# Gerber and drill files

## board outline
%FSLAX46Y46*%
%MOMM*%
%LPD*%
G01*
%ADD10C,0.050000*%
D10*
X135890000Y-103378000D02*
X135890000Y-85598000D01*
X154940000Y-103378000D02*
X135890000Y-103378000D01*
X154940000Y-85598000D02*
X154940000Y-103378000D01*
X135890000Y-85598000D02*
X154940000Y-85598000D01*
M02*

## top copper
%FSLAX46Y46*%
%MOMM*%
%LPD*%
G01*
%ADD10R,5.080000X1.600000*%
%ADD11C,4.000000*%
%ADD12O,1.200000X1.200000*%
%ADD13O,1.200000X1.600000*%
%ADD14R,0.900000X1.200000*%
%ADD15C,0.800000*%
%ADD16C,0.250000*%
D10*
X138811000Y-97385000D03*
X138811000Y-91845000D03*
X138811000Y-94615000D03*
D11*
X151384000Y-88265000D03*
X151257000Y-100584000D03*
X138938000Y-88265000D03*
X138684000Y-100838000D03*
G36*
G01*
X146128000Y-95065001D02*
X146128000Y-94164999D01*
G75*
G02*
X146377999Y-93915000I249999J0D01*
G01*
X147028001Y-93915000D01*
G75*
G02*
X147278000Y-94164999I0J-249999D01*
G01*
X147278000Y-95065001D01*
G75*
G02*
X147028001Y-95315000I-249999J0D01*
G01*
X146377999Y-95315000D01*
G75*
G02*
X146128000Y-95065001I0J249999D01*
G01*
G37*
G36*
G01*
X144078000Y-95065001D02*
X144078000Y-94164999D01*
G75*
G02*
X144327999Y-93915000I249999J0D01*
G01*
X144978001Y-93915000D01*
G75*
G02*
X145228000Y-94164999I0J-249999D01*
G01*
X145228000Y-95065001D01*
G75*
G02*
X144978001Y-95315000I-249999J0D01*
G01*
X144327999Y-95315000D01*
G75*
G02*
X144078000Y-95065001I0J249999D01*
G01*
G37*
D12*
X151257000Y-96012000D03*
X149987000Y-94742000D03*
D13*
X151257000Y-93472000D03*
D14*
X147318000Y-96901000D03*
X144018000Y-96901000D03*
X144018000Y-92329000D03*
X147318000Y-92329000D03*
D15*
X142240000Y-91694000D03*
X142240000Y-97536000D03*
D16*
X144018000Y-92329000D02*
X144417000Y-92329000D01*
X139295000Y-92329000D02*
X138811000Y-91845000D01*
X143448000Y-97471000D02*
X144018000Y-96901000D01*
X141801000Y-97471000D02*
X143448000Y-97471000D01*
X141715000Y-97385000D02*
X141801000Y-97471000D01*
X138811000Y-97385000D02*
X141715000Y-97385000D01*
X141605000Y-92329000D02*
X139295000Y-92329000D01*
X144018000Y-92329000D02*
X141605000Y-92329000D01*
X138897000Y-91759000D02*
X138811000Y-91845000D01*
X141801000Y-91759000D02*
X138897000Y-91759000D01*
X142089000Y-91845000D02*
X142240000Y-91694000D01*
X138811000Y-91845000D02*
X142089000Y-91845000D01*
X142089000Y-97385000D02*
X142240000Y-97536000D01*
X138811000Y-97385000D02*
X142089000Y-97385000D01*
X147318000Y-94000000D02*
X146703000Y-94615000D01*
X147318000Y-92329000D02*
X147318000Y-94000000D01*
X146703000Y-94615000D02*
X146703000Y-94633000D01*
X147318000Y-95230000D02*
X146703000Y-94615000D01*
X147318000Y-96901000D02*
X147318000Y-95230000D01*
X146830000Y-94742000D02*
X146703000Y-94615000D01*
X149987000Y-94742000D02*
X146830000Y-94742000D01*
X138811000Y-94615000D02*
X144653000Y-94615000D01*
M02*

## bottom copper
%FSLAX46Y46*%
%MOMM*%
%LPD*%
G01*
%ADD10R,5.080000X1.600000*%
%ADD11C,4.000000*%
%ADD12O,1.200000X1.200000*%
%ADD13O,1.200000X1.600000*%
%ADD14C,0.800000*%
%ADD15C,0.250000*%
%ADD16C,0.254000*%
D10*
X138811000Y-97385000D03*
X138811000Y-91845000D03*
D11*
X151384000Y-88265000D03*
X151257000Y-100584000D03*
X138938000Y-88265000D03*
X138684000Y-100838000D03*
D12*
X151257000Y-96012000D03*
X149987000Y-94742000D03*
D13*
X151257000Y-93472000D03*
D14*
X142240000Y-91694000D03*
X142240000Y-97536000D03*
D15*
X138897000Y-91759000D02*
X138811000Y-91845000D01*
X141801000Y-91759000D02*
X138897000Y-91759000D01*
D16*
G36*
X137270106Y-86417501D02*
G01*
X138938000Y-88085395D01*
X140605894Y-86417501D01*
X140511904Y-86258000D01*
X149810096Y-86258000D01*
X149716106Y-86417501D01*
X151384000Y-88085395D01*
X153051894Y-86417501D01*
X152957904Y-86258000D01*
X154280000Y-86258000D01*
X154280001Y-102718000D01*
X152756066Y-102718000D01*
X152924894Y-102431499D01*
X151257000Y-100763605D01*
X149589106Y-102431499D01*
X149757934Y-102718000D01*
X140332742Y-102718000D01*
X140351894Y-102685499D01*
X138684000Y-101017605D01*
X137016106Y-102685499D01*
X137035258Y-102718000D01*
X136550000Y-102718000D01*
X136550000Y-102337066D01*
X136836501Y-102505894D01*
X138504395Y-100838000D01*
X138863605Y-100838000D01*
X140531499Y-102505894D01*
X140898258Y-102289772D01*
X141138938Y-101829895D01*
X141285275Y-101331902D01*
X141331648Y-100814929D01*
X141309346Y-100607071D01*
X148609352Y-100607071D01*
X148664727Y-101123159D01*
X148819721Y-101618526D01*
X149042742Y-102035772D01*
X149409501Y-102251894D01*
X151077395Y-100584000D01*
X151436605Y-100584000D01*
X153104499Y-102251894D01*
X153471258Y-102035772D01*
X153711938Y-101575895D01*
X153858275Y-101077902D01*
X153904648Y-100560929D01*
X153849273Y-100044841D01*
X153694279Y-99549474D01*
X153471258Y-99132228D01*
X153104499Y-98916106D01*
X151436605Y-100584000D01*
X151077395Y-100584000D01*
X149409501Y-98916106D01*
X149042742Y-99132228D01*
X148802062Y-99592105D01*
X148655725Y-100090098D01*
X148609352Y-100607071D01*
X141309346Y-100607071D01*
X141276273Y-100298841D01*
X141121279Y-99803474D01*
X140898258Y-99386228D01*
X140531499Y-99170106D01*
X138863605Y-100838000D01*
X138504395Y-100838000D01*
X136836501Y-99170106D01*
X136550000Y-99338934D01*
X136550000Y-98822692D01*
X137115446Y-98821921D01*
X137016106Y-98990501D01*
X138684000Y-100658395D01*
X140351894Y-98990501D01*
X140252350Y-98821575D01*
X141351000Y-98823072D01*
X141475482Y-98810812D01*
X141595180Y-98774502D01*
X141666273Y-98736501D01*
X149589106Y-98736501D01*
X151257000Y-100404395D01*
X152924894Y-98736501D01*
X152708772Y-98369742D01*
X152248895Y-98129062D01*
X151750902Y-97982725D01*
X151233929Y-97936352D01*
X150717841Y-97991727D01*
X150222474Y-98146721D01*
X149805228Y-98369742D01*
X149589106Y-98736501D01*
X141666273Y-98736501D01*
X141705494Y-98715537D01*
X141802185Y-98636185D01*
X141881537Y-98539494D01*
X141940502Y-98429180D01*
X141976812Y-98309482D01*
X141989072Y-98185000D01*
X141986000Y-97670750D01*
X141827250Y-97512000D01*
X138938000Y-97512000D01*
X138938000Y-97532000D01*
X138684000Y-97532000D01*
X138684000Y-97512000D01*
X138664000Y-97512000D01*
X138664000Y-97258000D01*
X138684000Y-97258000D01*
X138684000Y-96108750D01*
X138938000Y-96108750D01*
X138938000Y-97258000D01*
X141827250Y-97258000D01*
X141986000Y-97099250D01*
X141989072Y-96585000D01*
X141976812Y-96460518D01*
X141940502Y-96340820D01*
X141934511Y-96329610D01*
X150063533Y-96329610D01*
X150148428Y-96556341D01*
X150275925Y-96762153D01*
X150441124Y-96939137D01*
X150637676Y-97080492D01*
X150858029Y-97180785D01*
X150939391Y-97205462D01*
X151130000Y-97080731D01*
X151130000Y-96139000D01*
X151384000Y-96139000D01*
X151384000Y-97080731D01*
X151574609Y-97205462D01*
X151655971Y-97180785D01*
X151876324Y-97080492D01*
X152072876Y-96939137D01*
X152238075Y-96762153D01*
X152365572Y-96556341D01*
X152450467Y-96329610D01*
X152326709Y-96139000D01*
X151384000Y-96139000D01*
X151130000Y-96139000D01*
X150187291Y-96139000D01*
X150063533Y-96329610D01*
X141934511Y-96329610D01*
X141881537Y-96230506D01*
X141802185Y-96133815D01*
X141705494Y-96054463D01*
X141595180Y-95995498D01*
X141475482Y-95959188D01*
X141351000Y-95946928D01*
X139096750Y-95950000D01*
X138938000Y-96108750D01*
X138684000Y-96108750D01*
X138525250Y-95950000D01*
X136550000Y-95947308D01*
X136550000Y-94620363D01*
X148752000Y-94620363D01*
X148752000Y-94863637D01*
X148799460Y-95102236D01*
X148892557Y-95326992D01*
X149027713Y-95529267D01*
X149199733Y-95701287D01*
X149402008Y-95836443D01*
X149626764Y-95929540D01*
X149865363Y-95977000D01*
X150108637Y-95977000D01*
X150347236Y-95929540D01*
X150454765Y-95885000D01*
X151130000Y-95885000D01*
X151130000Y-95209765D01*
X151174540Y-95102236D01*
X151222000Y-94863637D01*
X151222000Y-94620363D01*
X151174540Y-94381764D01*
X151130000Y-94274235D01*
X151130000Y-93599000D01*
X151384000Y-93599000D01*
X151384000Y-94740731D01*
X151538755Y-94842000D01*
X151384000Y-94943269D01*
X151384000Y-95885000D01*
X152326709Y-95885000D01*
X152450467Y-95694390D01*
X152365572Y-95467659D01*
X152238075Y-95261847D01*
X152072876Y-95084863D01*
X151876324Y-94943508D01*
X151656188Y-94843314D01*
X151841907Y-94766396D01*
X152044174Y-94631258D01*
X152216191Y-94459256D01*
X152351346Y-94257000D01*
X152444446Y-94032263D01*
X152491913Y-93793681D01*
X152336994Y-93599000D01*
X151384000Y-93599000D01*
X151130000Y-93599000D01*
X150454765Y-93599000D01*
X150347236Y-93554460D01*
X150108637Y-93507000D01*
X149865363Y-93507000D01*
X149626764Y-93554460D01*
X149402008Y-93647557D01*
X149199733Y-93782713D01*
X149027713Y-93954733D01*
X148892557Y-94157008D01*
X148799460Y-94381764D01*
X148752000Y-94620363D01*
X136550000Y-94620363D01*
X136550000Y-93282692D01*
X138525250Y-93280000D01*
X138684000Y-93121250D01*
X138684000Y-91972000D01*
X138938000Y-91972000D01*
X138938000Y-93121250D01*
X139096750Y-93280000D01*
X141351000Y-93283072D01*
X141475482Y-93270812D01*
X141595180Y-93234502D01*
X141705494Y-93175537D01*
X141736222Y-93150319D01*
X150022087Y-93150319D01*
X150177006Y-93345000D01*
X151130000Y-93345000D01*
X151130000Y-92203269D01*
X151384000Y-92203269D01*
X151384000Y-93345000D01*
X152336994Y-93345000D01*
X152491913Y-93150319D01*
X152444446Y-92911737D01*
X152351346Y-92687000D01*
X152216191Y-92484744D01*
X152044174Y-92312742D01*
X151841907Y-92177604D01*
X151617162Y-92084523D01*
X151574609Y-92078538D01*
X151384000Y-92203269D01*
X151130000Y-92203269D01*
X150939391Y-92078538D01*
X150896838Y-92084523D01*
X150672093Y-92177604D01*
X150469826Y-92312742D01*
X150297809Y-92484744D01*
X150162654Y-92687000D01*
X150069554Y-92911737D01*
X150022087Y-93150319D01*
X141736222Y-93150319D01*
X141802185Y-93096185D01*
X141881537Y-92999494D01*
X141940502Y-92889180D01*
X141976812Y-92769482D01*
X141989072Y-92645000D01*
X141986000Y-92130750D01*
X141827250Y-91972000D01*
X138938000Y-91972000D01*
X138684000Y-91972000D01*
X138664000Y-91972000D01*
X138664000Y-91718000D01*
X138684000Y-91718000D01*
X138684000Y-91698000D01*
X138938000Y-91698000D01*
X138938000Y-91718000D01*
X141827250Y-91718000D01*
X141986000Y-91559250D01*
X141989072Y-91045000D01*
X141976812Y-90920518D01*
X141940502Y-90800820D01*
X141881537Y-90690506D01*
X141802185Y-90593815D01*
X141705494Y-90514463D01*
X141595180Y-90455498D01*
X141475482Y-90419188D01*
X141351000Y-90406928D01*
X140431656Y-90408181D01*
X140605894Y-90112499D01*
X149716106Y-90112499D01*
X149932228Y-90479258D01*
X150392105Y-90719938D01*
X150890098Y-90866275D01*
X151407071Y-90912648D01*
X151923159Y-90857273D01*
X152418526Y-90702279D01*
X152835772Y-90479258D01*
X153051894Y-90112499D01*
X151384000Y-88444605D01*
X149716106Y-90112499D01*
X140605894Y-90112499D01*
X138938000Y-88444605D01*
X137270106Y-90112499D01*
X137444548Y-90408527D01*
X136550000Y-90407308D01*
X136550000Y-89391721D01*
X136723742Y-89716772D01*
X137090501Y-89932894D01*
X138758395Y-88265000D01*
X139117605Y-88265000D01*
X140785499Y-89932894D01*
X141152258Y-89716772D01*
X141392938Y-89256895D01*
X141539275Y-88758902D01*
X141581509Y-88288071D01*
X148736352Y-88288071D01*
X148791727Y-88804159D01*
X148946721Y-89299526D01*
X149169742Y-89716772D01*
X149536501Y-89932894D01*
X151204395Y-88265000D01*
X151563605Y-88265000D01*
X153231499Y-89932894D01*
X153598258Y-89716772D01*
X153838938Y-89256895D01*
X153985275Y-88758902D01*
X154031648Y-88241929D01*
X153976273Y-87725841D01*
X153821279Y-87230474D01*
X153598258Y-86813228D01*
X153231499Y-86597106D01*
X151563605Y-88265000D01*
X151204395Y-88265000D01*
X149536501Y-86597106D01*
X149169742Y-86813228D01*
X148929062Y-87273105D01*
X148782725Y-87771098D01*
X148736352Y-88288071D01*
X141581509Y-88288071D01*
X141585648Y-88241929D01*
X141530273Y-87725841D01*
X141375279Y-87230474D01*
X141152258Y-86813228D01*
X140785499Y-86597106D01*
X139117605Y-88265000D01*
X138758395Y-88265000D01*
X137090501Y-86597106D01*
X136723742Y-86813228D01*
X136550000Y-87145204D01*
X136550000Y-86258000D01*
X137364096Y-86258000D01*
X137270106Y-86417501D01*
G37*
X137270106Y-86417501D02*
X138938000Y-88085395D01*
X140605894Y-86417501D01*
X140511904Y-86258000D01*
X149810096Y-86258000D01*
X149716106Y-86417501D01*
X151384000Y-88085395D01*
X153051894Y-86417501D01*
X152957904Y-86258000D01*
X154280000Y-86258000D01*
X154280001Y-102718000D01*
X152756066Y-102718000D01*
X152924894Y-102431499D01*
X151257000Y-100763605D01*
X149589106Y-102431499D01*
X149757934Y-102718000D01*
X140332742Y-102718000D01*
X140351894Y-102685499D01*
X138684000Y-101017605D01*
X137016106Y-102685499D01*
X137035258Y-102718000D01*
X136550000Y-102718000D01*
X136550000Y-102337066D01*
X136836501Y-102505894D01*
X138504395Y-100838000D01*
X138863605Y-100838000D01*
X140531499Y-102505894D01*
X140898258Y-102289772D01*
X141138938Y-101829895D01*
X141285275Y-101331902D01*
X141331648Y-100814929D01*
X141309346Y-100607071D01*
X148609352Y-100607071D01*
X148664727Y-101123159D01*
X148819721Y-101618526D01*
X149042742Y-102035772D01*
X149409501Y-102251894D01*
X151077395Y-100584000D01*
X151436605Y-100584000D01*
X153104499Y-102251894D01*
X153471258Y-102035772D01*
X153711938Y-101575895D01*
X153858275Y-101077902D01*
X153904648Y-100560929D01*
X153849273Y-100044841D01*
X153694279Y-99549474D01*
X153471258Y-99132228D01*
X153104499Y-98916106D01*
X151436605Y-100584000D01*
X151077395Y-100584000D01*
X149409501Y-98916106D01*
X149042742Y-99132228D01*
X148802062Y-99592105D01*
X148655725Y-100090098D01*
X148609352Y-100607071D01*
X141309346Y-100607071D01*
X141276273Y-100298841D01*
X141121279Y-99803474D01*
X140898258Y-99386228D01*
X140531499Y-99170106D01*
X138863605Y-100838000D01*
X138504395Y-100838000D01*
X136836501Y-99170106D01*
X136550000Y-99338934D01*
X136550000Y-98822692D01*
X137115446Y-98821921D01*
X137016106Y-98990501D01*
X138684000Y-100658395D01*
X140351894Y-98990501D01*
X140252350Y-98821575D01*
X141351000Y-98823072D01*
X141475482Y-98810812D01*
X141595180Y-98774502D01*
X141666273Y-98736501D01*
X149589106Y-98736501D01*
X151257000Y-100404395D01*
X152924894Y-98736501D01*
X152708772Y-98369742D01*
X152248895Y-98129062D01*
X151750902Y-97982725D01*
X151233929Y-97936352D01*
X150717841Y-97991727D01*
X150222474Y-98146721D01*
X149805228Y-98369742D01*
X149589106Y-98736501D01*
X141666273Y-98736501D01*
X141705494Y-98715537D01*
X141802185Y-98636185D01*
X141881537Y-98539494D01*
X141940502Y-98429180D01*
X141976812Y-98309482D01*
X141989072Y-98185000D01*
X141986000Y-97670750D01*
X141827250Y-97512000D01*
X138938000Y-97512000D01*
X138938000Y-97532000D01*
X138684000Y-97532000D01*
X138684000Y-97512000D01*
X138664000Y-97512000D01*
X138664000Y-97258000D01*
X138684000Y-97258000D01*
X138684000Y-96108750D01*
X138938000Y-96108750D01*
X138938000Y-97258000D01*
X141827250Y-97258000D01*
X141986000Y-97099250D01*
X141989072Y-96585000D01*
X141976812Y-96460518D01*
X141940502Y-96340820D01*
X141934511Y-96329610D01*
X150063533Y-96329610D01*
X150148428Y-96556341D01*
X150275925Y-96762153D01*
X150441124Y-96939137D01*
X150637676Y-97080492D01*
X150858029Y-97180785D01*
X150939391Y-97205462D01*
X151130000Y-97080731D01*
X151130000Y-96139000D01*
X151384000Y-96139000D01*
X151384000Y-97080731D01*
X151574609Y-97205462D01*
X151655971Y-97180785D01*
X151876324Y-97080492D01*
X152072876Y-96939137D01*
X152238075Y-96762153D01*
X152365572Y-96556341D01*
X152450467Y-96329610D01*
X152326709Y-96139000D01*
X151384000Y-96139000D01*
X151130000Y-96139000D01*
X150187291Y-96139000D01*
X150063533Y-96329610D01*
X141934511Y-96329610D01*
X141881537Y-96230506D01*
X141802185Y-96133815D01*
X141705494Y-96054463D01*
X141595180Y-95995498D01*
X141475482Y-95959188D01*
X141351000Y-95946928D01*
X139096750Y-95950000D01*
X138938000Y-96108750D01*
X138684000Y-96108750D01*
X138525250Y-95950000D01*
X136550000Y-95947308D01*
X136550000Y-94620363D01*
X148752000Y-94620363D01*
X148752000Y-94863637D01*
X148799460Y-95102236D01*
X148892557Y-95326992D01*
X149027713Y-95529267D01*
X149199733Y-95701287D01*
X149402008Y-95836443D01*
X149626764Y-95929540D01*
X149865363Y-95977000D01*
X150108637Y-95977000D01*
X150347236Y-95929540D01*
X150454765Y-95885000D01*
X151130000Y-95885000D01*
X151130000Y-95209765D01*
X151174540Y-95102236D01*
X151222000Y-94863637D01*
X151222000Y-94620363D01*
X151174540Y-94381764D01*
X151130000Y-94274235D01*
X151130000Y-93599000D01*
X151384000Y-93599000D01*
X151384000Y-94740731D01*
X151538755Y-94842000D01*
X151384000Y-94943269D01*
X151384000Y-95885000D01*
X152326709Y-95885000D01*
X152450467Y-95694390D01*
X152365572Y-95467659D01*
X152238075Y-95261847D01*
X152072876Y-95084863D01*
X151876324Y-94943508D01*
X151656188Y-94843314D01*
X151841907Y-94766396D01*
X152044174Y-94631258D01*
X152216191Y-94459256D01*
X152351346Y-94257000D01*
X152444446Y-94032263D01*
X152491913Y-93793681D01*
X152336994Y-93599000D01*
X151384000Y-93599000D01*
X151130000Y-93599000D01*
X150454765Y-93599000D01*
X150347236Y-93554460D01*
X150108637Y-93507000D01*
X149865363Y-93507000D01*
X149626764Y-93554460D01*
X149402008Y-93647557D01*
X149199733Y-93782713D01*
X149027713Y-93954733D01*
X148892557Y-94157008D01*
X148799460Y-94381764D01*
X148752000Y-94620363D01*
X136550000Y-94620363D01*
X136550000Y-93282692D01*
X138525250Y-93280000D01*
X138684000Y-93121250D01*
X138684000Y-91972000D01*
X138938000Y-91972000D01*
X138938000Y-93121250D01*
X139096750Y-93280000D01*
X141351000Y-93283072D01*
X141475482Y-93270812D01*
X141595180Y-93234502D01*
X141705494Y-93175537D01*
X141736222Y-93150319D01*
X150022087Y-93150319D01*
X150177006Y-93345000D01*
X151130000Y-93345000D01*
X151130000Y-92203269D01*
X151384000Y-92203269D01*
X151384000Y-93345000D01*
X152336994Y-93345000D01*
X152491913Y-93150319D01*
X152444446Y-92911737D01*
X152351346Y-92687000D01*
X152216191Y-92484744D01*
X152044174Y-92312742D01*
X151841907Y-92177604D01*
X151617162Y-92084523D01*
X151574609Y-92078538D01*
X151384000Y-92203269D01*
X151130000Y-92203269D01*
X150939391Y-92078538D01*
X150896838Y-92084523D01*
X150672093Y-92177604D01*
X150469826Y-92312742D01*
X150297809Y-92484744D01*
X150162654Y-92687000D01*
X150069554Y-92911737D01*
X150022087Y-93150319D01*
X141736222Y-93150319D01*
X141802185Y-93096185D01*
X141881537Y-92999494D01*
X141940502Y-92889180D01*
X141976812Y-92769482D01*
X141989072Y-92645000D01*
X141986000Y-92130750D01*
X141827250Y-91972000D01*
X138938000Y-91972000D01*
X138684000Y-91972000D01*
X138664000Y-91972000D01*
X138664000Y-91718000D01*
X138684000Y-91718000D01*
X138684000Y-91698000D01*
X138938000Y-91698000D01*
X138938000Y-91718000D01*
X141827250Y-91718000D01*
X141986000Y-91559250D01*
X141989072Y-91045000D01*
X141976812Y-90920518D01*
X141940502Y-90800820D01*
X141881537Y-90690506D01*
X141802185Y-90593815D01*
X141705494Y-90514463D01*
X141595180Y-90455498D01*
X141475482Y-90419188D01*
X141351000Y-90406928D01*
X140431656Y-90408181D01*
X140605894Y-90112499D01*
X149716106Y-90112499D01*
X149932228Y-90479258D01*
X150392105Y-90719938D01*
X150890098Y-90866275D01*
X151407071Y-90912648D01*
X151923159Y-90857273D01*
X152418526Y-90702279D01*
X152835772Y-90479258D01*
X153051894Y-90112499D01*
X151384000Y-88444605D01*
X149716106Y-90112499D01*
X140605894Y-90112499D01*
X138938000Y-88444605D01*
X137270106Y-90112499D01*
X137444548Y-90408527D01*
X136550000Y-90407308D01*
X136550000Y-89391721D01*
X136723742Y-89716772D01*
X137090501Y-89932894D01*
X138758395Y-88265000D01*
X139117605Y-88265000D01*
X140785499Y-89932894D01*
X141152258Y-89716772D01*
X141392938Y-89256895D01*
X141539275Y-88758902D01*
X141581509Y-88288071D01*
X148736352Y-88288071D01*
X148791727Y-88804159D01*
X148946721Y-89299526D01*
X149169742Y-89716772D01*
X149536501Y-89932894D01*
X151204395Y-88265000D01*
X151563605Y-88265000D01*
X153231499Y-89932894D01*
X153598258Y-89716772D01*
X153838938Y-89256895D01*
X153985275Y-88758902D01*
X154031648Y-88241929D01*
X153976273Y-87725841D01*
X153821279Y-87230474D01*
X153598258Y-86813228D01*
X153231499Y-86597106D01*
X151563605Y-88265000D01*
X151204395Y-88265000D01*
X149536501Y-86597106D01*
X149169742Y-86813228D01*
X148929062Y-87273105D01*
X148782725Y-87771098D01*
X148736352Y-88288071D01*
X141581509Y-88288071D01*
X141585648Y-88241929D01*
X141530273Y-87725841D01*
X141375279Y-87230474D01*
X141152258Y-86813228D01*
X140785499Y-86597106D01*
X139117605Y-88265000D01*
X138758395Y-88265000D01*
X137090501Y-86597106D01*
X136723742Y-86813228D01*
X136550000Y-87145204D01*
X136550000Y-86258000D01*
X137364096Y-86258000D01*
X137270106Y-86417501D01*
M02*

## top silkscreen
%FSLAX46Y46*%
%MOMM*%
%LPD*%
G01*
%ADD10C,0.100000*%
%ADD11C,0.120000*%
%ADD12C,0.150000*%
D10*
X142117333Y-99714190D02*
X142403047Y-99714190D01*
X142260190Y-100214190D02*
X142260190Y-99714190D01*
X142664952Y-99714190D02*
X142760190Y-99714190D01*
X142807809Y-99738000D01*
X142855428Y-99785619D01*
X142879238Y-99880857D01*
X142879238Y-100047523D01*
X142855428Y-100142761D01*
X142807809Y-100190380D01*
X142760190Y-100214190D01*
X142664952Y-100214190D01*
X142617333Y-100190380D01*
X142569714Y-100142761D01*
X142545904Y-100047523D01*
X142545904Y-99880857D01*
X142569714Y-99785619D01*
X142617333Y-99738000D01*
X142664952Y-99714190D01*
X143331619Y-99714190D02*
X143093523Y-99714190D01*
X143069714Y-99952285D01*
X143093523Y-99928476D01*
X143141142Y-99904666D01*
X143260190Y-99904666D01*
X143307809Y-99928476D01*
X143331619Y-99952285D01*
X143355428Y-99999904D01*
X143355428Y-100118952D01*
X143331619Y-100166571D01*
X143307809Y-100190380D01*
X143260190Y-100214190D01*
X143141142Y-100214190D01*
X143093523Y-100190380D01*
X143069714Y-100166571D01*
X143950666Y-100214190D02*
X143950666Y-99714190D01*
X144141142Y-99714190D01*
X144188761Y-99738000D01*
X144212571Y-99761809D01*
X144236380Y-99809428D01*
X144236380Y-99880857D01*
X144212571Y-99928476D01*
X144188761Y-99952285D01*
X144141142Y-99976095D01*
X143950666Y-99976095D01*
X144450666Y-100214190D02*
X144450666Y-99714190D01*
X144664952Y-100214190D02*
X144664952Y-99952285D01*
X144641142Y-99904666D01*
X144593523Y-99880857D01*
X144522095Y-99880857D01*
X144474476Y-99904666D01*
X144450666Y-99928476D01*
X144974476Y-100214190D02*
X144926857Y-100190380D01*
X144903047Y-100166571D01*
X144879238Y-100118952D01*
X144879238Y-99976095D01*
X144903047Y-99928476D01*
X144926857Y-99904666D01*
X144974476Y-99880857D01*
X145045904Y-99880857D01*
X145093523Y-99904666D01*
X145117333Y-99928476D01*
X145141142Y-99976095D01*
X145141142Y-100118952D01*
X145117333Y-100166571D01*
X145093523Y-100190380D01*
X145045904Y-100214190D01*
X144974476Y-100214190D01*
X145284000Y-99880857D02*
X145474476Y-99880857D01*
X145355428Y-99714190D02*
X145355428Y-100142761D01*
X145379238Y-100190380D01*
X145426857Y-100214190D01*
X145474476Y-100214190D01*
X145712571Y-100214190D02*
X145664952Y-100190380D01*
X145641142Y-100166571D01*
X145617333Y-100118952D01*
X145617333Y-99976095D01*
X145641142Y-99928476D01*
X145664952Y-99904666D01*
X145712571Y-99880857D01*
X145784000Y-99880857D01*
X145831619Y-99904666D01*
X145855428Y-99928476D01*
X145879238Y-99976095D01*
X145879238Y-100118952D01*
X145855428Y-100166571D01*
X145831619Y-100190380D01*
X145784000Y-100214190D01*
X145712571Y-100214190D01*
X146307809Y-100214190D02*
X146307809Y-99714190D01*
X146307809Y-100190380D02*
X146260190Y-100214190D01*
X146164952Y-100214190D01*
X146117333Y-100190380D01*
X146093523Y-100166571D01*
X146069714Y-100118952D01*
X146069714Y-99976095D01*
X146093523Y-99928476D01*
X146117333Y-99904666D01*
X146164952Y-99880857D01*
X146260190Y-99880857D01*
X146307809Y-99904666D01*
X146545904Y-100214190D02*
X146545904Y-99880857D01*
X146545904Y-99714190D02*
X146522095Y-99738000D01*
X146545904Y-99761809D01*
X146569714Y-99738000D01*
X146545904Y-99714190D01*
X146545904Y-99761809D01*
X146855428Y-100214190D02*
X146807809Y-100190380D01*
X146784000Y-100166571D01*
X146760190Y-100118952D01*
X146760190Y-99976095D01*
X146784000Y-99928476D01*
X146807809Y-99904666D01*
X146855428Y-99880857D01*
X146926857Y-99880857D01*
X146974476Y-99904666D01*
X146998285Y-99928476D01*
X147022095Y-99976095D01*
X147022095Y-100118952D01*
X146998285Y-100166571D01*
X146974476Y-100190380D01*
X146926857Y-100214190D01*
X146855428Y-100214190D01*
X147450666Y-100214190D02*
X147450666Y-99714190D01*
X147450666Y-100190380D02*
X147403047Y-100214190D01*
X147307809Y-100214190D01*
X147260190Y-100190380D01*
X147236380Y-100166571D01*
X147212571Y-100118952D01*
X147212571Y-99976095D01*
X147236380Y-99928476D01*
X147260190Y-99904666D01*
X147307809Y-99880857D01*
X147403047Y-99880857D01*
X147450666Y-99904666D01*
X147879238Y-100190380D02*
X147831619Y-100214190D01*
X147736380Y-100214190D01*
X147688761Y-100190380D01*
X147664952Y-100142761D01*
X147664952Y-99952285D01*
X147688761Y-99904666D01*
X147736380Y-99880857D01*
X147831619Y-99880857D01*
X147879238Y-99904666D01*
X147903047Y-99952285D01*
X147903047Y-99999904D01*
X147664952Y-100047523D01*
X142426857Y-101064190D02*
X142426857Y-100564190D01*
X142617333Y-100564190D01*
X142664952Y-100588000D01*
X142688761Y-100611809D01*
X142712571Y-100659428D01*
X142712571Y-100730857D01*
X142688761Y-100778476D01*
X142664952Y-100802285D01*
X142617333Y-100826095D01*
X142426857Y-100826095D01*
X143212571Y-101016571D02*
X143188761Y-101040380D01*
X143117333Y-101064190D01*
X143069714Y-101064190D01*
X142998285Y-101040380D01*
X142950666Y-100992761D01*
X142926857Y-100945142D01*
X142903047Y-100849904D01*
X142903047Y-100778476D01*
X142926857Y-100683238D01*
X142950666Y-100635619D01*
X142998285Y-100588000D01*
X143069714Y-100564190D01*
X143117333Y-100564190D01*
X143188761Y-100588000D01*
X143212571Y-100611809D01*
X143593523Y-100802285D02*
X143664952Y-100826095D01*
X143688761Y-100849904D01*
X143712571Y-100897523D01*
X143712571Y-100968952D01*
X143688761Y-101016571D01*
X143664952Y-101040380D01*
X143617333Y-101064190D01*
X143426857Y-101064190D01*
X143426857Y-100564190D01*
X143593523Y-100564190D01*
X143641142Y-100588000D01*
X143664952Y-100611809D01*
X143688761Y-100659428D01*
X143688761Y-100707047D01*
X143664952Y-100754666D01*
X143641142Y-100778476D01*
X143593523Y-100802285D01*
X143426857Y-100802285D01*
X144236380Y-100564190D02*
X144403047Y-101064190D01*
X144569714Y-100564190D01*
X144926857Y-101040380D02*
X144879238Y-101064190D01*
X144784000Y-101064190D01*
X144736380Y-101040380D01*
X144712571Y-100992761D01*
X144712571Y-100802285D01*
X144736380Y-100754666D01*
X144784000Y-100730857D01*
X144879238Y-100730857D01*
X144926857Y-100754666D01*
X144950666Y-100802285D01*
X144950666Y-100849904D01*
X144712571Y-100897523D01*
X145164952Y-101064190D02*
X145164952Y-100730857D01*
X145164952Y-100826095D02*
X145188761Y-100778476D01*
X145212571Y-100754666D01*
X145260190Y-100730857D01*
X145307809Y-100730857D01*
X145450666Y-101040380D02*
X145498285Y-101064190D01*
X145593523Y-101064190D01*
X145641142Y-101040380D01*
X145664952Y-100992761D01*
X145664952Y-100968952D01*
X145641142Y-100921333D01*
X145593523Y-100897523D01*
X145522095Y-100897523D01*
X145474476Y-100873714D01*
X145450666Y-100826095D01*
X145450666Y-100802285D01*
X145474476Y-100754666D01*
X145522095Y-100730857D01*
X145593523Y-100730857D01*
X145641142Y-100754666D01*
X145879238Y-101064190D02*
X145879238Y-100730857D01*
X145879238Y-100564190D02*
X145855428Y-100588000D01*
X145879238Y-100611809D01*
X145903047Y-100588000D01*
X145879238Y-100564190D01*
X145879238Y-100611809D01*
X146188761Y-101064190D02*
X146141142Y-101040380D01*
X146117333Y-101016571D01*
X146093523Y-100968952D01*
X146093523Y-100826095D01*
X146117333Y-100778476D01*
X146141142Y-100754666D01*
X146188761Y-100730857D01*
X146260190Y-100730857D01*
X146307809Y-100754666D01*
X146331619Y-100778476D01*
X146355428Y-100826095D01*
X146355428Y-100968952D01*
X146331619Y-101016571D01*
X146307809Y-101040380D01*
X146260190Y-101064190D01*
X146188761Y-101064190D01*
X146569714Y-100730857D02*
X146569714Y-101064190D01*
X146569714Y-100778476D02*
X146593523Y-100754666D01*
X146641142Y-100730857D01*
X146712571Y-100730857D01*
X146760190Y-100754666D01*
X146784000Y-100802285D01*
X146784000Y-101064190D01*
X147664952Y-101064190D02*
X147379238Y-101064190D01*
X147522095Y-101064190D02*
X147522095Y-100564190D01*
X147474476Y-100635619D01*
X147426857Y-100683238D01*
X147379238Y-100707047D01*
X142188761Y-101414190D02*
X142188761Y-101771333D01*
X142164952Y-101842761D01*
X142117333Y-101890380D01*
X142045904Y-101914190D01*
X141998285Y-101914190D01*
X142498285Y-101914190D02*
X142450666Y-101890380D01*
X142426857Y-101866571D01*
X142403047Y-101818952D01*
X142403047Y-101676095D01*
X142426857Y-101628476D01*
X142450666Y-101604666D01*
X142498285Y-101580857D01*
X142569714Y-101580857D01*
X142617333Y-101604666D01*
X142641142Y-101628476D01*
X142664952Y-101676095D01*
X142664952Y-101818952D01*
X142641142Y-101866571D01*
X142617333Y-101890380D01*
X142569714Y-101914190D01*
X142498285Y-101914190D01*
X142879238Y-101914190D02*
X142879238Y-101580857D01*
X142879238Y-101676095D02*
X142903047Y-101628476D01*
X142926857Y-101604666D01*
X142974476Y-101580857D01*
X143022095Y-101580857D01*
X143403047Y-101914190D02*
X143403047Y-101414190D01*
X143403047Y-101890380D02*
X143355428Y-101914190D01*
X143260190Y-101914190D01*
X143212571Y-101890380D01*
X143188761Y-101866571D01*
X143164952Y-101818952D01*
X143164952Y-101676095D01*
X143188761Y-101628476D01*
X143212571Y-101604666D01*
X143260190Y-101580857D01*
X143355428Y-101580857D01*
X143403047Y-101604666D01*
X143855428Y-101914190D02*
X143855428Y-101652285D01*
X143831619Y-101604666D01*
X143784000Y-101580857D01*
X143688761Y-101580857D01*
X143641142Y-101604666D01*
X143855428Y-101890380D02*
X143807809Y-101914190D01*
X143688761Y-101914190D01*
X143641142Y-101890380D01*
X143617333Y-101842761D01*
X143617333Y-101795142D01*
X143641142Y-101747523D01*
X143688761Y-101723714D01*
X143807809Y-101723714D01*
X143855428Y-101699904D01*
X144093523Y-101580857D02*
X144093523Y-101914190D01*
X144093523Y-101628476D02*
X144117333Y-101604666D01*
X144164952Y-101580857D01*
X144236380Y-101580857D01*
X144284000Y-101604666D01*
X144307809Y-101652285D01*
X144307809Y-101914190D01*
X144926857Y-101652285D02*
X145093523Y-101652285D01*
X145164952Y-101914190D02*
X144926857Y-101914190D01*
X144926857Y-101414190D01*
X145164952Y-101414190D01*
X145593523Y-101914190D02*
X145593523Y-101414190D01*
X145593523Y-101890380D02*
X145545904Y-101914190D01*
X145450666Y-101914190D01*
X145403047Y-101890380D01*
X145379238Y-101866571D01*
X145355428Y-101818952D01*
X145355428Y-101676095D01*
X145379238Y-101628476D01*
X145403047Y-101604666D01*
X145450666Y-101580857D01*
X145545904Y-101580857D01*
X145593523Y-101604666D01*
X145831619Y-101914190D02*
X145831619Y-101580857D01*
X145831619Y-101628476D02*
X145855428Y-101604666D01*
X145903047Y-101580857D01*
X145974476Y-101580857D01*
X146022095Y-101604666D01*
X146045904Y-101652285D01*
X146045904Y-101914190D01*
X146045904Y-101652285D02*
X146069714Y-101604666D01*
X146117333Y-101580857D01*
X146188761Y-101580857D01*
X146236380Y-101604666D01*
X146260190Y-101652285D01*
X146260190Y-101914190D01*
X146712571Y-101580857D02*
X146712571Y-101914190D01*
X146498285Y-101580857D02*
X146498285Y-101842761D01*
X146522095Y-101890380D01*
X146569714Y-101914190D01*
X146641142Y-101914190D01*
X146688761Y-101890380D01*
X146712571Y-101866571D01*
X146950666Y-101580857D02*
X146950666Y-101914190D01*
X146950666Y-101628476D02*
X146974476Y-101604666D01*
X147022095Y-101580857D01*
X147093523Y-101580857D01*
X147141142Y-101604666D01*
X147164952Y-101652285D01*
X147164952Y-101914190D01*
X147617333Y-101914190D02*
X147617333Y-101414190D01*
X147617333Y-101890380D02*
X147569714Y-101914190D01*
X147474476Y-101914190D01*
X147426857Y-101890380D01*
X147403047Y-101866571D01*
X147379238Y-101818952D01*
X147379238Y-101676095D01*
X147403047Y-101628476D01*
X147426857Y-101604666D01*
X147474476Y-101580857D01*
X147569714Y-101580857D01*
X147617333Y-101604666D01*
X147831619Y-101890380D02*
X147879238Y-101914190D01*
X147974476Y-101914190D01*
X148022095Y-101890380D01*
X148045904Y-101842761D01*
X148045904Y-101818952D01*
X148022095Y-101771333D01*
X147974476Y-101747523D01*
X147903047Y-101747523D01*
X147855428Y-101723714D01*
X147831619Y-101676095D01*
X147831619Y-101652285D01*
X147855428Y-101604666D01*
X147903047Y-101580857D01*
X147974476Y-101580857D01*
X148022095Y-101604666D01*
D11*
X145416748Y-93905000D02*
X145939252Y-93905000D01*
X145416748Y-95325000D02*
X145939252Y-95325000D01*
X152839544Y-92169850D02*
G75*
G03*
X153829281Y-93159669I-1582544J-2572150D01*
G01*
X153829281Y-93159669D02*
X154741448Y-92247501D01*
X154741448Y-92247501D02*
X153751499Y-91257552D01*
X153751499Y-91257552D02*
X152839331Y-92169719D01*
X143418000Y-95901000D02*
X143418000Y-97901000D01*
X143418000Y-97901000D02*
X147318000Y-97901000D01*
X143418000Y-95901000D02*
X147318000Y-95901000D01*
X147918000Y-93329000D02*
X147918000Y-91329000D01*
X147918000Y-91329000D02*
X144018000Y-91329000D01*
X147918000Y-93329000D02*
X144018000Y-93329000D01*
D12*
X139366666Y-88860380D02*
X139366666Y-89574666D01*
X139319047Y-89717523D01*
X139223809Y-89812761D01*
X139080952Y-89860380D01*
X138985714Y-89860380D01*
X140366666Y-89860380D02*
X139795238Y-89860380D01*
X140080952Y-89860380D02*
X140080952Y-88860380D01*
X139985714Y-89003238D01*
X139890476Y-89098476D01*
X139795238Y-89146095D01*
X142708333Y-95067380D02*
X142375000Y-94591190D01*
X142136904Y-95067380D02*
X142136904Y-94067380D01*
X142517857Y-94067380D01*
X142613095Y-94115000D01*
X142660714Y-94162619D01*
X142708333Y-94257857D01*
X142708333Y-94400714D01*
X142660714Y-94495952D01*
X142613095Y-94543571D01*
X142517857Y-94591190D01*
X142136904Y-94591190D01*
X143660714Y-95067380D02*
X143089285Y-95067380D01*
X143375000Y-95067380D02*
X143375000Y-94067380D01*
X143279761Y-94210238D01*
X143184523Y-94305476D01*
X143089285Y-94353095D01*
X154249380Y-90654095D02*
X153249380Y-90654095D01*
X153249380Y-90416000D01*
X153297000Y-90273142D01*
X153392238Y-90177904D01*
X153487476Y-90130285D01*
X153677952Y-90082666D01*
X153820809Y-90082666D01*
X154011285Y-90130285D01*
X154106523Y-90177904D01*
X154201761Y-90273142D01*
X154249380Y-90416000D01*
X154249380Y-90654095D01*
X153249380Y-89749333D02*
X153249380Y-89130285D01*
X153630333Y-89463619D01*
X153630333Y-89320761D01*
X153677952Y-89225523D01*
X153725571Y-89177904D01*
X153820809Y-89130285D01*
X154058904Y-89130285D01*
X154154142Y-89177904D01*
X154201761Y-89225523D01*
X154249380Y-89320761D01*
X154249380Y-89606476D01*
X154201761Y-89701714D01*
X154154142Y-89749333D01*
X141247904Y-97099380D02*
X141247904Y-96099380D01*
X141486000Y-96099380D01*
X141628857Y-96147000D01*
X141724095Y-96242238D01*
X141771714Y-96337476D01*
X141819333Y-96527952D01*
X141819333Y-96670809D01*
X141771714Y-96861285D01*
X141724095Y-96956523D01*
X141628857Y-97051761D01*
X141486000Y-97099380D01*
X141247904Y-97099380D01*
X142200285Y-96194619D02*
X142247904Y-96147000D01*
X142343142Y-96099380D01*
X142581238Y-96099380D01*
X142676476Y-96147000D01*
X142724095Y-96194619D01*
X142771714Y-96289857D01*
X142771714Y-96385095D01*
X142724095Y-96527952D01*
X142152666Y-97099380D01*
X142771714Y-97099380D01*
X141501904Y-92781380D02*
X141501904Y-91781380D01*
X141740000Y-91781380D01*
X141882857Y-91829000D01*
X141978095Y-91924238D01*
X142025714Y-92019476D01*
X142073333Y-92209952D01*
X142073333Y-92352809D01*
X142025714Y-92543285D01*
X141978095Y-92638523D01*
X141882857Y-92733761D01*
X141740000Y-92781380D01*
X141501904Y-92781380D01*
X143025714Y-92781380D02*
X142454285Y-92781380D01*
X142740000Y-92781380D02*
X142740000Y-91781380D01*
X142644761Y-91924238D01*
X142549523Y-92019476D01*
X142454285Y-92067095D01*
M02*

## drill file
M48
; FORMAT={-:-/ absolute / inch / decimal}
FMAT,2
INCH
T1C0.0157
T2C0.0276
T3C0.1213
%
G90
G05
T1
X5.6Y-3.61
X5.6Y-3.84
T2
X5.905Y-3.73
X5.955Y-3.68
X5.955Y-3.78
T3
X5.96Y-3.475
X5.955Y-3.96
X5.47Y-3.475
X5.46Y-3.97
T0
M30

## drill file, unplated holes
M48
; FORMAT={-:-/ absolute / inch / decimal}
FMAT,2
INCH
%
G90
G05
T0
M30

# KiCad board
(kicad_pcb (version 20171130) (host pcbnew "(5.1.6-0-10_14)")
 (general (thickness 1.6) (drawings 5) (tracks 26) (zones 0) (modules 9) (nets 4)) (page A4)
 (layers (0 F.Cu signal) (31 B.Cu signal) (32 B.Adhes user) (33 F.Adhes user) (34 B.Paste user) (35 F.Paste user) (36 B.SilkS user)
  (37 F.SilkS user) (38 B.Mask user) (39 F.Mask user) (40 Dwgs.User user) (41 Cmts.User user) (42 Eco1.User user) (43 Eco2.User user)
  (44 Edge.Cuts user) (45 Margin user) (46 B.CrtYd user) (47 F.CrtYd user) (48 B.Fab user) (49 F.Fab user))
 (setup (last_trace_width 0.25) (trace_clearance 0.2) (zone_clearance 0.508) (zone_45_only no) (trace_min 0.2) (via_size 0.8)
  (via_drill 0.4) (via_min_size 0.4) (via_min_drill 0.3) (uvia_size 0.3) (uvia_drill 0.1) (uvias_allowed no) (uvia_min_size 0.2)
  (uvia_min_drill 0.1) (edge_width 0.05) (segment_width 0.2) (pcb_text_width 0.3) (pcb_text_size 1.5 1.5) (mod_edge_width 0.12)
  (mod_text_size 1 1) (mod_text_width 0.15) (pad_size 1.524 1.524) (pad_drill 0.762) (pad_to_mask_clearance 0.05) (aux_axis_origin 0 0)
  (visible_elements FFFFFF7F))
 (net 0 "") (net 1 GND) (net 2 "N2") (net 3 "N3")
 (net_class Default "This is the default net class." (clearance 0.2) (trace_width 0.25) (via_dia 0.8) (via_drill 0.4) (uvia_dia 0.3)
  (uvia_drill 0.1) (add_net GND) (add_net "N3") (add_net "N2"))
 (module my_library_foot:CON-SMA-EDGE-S (layer F.Cu) (at 140.531 94.615)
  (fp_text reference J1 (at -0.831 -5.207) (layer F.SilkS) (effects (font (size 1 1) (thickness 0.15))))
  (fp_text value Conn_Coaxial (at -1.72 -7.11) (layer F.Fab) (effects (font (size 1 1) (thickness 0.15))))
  (pad 2 smd rect (at -1.72 2.77) (size 5.08 1.6) (layers B.Cu B.Paste B.Mask) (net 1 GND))
  (pad 2 smd rect (at -1.72 -2.77) (size 5.08 1.6) (layers B.Cu B.Paste B.Mask) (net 1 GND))
  (pad 2 smd rect (at -1.72 2.77) (size 5.08 1.6) (layers F.Cu F.Paste F.Mask) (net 1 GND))
  (pad 2 smd rect (at -1.72 -2.77) (size 5.08 1.6) (layers F.Cu F.Paste F.Mask) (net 1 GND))
  (pad 1 smd rect (at -1.72 0) (size 5.08 1.6) (layers F.Cu F.Paste F.Mask) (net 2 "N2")))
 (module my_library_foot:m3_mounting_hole (layer F.Cu) (at 151.384 88.265)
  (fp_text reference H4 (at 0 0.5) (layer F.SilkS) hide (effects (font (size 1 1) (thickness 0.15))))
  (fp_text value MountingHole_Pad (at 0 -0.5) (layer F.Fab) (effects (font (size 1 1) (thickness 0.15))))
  (pad 1 thru_hole circle (at 0 0) (size 4 4) (drill 3.08) (layers *.Cu *.Mask) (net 1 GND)))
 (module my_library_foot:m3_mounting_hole (layer F.Cu) (at 151.257 100.584)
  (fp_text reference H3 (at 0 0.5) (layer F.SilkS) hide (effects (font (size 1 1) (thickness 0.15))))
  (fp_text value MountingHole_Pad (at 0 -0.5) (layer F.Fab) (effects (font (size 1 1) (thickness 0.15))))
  (pad 1 thru_hole circle (at 0 0) (size 4 4) (drill 3.08) (layers *.Cu *.Mask) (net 1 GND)))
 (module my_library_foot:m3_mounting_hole (layer F.Cu) (at 138.938 88.265)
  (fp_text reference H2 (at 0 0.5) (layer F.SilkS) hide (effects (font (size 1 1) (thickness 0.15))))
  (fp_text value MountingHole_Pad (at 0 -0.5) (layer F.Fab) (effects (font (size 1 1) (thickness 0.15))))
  (pad 1 thru_hole circle (at 0 0) (size 4 4) (drill 3.08) (layers *.Cu *.Mask) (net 1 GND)))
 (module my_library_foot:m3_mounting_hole (layer F.Cu) (at 138.684 100.838)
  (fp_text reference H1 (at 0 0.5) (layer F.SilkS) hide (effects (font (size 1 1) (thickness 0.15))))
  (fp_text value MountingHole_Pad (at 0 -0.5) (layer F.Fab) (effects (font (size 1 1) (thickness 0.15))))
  (pad 1 thru_hole circle (at 0 0) (size 4 4) (drill 3.08) (layers *.Cu *.Mask) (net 1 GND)))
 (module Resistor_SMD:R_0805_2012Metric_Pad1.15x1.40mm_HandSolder (layer F.Cu) (at 145.678 94.615)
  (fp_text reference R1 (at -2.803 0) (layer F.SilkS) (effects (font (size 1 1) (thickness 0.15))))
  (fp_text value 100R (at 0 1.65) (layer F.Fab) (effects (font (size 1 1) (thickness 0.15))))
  (fp_line (start -0.261252 -0.71) (end 0.261252 -0.71) (layer F.SilkS) (width 0.12))
  (fp_line (start -0.261252 0.71) (end 0.261252 0.71) (layer F.SilkS) (width 0.12))
  (pad 2 smd roundrect (at 1.025 0) (size 1.15 1.4) (layers F.Cu F.Paste F.Mask) (roundrect_rratio 0.217391) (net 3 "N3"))
  (pad 1 smd roundrect (at -1.025 0) (size 1.15 1.4) (layers F.Cu F.Paste F.Mask) (roundrect_rratio 0.217391) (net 2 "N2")))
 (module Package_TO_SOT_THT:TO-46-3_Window (layer F.Cu) (at 151.257 93.472 270)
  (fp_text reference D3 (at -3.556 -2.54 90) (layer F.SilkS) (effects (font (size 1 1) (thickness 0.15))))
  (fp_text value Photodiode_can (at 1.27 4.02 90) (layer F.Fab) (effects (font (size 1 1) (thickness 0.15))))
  (fp_arc (start 1.27 0) (end -0.312331 -2.572281) (angle 333.2) (layer F.SilkS) (width 0.12))
  (fp_line (start -0.312331 -2.572281) (end -1.224499 -3.484448) (layer F.SilkS) (width 0.12))
  (fp_line (start -1.224499 -3.484448) (end -2.214448 -2.494499) (layer F.SilkS) (width 0.12))
  (fp_line (start -2.214448 -2.494499) (end -1.302281 -1.582331) (layer F.SilkS) (width 0.12))
  (pad 3 thru_hole oval (at 2.54 0 270) (size 1.2 1.2) (drill 0.7) (layers *.Cu *.Mask) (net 1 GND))
  (pad 2 thru_hole oval (at 1.27 1.27 270) (size 1.2 1.2) (drill 0.7) (layers *.Cu *.Mask) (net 3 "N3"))
  (pad 1 thru_hole oval (at 0 0 270) (size 1.6 1.2) (drill 0.7) (layers *.Cu *.Mask) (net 1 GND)))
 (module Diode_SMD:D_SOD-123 (layer F.Cu) (at 145.668 96.901)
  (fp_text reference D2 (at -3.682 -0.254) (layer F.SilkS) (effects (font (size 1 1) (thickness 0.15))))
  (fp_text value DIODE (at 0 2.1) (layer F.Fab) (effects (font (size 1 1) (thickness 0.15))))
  (fp_line (start -2.25 -1) (end -2.25 1) (layer F.SilkS) (width 0.12))
  (fp_line (start -2.25 1) (end 1.65 1) (layer F.SilkS) (width 0.12))
  (fp_line (start -2.25 -1) (end 1.65 -1) (layer F.SilkS) (width 0.12))
  (pad 2 smd rect (at 1.65 0) (size 0.9 1.2) (layers F.Cu F.Paste F.Mask) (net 3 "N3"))
  (pad 1 smd rect (at -1.65 0) (size 0.9 1.2) (layers F.Cu F.Paste F.Mask) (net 1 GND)))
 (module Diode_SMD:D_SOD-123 (layer F.Cu) (at 145.668 92.329 180)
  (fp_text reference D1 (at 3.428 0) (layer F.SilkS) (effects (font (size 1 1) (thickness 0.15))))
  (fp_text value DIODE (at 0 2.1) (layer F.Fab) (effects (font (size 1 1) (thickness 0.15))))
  (fp_line (start -2.25 -1) (end -2.25 1) (layer F.SilkS) (width 0.12))
  (fp_line (start -2.25 1) (end 1.65 1) (layer F.SilkS) (width 0.12))
  (fp_line (start -2.25 -1) (end 1.65 -1) (layer F.SilkS) (width 0.12))
  (pad 2 smd rect (at 1.65 0 180) (size 0.9 1.2) (layers F.Cu F.Paste F.Mask) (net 1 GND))
  (pad 1 smd rect (at -1.65 0 180) (size 0.9 1.2) (layers F.Cu F.Paste F.Mask) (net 3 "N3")))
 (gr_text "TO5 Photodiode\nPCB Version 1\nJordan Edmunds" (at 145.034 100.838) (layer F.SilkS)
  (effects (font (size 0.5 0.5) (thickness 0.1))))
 (gr_line (start 135.89 103.378) (end 135.89 85.598) (layer Edge.Cuts) (width 0.05))
 (gr_line (start 154.94 103.378) (end 135.89 103.378) (layer Edge.Cuts) (width 0.05))
 (gr_line (start 154.94 85.598) (end 154.94 103.378) (layer Edge.Cuts) (width 0.05))
 (gr_line (start 135.89 85.598) (end 154.94 85.598) (layer Edge.Cuts) (width 0.05))
 (segment (start 144.018 92.329) (end 144.417 92.329) (width 0.25) (layer F.Cu) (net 1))
 (segment (start 139.295 92.329) (end 138.811 91.845) (width 0.25) (layer F.Cu) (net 1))
 (segment (start 143.448 97.471) (end 144.018 96.901) (width 0.25) (layer F.Cu) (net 1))
 (segment (start 141.801 97.471) (end 143.448 97.471) (width 0.25) (layer F.Cu) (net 1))
 (segment (start 141.715 97.385) (end 141.801 97.471) (width 0.25) (layer F.Cu) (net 1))
 (segment (start 138.811 97.385) (end 141.715 97.385) (width 0.25) (layer F.Cu) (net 1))
 (segment (start 141.605 92.329) (end 139.295 92.329) (width 0.25) (layer F.Cu) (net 1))
 (segment (start 144.018 92.329) (end 141.605 92.329) (width 0.25) (layer F.Cu) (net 1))
 (segment (start 138.897 91.759) (end 138.811 91.845) (width 0.25) (layer F.Cu) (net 1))
 (segment (start 141.801 91.759) (end 138.897 91.759) (width 0.25) (layer F.Cu) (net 1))
 (segment (start 138.897 91.759) (end 138.811 91.845) (width 0.25) (layer B.Cu) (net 1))
 (segment (start 141.801 91.759) (end 138.897 91.759) (width 0.25) (layer B.Cu) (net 1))
 (via (at 142.24 91.694) (size 0.8) (drill 0.4) (layers F.Cu B.Cu) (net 1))
 (segment (start 142.089 91.845) (end 142.24 91.694) (width 0.25) (layer F.Cu) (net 1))
 (segment (start 138.811 91.845) (end 142.089 91.845) (width 0.25) (layer F.Cu) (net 1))
 (via (at 142.24 97.536) (size 0.8) (drill 0.4) (layers F.Cu B.Cu) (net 1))
 (segment (start 142.089 97.385) (end 142.24 97.536) (width 0.25) (layer F.Cu) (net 1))
 (segment (start 138.811 97.385) (end 142.089 97.385) (width 0.25) (layer F.Cu) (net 1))
 (segment (start 147.318 94) (end 146.703 94.615) (width 0.25) (layer F.Cu) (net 3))
 (segment (start 147.318 92.329) (end 147.318 94) (width 0.25) (layer F.Cu) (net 3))
 (segment (start 146.703 94.615) (end 146.703 94.633) (width 0.25) (layer F.Cu) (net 3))
 (segment (start 147.318 95.23) (end 146.703 94.615) (width 0.25) (layer F.Cu) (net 3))
 (segment (start 147.318 96.901) (end 147.318 95.23) (width 0.25) (layer F.Cu) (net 3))
 (segment (start 146.83 94.742) (end 146.703 94.615) (width 0.25) (layer F.Cu) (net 3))
 (segment (start 149.987 94.742) (end 146.83 94.742) (width 0.25) (layer F.Cu) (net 3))
 (segment (start 138.811 94.615) (end 144.653 94.615) (width 0.25) (layer F.Cu) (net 2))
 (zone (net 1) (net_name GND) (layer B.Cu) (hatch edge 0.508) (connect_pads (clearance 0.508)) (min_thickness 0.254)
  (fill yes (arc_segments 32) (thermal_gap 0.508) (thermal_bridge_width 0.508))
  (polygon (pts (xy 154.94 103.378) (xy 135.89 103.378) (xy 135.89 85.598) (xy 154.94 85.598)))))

